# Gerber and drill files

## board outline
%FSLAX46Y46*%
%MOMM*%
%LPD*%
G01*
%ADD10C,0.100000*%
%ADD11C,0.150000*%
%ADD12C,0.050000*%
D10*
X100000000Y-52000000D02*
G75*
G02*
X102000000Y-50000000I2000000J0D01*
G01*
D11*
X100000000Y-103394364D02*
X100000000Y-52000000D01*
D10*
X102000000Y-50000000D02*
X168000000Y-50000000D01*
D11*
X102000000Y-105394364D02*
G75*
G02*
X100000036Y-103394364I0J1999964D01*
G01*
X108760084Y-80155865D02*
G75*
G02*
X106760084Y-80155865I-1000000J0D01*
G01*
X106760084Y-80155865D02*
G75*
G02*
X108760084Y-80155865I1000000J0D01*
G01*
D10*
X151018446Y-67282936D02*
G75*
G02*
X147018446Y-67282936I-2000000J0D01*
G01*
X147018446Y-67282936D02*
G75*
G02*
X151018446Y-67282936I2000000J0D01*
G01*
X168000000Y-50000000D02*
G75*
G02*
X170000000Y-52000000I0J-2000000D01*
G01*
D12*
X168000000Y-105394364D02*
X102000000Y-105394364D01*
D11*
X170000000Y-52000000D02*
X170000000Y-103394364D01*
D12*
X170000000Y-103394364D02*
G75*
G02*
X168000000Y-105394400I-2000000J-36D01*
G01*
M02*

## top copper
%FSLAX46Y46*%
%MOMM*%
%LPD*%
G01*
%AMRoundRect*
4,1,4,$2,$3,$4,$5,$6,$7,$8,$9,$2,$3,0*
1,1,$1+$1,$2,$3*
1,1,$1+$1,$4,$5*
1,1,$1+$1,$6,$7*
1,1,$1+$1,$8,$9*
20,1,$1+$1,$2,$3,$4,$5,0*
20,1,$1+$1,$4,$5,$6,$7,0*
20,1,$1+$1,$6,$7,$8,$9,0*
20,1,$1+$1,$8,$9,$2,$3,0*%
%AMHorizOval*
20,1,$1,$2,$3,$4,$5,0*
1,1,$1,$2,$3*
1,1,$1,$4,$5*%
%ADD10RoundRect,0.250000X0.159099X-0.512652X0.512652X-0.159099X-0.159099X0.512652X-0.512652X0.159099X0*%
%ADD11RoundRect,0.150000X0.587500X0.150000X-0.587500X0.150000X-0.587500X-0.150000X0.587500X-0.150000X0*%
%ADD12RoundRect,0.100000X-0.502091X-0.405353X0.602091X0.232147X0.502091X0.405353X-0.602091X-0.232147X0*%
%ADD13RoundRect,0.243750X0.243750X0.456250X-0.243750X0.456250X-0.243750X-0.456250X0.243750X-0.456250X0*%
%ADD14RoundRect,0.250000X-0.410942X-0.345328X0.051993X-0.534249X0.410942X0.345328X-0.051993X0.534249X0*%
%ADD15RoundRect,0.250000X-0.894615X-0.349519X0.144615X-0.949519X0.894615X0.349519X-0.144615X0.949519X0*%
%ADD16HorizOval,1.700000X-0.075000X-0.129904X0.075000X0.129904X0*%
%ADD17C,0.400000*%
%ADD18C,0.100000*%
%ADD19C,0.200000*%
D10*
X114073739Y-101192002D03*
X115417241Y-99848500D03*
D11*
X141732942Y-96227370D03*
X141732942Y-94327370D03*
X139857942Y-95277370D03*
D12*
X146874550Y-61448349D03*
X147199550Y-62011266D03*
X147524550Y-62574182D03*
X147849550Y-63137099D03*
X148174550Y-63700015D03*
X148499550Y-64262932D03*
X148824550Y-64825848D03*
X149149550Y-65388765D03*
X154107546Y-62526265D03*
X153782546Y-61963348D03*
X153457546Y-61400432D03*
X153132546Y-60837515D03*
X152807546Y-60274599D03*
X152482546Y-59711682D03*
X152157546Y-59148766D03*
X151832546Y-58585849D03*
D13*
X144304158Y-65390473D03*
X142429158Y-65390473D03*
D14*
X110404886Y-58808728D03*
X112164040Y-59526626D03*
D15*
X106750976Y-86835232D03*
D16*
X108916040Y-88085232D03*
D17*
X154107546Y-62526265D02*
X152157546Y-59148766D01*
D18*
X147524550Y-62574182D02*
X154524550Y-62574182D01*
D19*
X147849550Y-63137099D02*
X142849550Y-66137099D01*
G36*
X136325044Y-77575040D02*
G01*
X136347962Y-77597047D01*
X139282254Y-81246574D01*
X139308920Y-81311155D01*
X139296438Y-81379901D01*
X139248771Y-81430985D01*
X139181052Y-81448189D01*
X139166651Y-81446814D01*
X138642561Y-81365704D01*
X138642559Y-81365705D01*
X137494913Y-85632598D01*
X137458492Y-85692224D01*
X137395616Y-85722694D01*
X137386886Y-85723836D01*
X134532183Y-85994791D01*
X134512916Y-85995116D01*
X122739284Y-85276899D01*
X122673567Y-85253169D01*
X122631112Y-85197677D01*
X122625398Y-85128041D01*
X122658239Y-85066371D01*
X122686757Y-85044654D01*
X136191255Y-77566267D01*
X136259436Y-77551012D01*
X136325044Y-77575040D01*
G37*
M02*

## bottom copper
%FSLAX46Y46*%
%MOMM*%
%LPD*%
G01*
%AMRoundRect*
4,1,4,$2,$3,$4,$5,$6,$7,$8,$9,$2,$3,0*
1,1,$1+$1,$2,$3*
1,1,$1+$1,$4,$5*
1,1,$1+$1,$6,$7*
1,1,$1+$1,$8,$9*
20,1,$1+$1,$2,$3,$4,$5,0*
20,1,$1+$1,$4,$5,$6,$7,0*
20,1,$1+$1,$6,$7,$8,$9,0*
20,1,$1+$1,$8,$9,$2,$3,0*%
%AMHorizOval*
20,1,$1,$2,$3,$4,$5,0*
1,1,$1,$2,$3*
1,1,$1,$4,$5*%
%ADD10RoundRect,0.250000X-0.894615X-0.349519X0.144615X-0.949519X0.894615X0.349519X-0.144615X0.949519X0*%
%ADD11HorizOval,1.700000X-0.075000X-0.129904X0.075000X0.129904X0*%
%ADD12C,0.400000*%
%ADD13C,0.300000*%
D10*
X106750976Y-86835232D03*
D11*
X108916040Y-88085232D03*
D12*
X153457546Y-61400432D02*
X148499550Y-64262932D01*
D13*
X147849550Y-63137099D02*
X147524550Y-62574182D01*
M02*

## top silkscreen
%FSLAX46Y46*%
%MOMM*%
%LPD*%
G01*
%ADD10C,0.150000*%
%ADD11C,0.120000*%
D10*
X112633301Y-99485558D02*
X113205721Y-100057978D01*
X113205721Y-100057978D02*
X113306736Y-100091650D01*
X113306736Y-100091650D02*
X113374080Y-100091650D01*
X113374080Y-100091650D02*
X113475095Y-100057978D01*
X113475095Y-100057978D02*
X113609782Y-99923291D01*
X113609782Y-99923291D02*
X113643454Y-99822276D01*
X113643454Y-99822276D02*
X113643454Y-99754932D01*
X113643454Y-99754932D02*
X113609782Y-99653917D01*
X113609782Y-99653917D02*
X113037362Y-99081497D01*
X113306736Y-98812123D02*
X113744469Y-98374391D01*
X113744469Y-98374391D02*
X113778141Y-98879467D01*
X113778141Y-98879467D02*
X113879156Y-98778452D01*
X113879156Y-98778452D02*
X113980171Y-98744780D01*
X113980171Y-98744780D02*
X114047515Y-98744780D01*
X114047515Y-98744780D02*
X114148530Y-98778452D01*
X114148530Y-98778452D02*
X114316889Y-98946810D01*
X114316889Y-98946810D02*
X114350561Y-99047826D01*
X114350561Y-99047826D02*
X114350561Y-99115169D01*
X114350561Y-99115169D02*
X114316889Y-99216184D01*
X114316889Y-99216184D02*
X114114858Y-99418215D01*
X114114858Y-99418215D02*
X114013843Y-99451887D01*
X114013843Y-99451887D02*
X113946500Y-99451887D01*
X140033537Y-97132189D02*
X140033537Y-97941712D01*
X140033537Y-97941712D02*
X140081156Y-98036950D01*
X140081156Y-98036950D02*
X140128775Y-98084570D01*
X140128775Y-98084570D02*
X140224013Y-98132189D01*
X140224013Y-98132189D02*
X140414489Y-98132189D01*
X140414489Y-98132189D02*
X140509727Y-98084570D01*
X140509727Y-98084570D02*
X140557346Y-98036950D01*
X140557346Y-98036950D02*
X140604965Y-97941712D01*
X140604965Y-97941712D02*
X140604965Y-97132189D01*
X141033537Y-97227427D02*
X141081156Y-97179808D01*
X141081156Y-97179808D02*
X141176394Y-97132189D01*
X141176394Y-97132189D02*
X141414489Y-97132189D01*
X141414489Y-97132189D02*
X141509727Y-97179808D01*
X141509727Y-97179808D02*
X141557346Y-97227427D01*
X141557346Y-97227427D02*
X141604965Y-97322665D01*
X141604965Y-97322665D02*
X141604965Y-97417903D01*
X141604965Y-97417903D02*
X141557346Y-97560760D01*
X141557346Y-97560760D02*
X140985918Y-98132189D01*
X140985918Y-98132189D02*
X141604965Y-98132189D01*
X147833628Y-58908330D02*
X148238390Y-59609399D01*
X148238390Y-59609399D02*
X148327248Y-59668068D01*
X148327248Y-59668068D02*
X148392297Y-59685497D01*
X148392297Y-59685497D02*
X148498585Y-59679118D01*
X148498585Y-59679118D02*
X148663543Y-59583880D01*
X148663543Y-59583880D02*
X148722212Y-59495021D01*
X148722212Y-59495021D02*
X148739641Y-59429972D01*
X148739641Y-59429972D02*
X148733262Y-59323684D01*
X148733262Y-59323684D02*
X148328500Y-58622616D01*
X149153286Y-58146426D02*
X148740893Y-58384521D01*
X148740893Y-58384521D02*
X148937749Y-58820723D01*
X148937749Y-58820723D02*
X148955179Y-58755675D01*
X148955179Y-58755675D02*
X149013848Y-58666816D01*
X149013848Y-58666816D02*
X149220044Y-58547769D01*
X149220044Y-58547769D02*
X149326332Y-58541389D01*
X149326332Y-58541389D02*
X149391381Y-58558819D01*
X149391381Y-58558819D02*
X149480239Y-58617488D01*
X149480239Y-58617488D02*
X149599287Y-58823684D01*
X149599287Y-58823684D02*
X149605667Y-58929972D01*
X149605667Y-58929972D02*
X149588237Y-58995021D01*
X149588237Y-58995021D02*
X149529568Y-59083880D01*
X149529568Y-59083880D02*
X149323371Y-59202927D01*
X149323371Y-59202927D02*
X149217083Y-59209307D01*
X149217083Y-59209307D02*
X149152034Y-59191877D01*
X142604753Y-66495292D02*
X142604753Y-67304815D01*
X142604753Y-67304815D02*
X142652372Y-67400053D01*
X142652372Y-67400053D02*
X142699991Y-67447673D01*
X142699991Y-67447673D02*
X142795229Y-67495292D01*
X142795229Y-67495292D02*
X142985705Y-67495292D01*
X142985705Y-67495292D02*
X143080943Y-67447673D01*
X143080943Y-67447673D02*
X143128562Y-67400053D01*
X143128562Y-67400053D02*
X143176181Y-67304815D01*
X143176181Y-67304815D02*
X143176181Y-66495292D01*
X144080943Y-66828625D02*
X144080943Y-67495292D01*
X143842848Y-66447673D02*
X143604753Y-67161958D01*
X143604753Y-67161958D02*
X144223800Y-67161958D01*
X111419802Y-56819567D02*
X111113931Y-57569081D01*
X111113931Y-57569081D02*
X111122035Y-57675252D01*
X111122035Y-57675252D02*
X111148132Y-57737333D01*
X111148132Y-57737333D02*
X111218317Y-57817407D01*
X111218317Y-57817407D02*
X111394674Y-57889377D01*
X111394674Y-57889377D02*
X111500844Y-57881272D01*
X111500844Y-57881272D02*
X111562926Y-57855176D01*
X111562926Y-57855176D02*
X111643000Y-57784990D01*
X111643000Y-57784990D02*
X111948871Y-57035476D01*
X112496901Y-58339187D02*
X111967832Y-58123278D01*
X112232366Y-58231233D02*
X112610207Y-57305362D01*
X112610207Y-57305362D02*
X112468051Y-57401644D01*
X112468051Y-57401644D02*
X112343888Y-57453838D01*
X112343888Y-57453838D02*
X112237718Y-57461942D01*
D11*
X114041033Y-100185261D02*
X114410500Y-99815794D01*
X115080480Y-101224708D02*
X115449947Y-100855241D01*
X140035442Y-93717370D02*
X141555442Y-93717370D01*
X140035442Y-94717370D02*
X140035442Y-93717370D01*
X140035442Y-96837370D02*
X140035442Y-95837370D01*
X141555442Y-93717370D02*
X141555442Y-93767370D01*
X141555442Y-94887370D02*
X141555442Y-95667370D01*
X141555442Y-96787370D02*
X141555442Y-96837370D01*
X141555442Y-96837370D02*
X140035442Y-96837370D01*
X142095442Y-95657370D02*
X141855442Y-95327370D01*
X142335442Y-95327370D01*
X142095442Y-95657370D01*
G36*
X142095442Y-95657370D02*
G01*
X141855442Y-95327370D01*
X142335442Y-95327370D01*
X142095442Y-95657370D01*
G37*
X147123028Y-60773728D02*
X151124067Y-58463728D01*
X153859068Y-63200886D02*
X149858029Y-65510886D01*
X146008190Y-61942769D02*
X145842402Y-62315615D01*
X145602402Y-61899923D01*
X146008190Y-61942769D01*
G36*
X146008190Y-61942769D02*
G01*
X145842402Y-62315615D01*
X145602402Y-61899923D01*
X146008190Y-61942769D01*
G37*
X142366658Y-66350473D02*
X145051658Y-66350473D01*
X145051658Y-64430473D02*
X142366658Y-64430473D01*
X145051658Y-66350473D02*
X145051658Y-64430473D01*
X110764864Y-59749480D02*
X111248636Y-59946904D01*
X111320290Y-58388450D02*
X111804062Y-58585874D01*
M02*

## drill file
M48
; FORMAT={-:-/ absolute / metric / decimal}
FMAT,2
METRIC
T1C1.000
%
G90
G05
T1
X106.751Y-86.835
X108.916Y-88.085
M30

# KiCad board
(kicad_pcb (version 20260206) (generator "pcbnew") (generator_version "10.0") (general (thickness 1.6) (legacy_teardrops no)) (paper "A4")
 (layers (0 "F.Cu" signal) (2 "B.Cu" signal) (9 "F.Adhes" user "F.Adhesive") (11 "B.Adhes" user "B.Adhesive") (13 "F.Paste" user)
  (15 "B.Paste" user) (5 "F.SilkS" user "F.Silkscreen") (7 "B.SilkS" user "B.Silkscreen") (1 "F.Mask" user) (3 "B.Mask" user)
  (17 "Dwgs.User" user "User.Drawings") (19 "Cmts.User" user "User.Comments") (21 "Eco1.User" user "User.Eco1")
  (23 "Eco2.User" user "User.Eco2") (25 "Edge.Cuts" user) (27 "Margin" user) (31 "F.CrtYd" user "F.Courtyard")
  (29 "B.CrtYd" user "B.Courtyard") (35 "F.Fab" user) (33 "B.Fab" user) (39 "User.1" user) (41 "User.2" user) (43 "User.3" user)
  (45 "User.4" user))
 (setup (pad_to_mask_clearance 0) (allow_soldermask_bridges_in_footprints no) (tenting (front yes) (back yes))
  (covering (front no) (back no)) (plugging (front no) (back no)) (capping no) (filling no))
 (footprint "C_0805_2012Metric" (layer "F.Cu") (at 114.74549 100.520251 45)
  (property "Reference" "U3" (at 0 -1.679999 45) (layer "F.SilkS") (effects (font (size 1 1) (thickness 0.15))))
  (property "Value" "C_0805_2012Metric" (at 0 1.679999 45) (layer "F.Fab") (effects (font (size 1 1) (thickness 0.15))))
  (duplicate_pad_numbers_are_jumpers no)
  (fp_line (start -0.261253 -0.735) (end 0.261253 -0.735) (stroke (width 0.12) (type solid)) (layer "F.SilkS"))
  (fp_line (start -0.261253 0.735) (end 0.261253 0.735) (stroke (width 0.12) (type solid)) (layer "F.SilkS"))
  (pad "1" smd roundrect (at -0.949999 0 45) (size 1 1.45) (layers "F.Cu" "F.Mask" "F.Paste") (roundrect_rratio 0.25) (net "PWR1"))
  (pad "2" smd roundrect (at 0.949999 0 45) (size 1 1.45) (layers "F.Cu" "F.Mask" "F.Paste") (roundrect_rratio 0.25) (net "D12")))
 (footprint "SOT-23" (layer "F.Cu") (at 140.795442 95.27737 180)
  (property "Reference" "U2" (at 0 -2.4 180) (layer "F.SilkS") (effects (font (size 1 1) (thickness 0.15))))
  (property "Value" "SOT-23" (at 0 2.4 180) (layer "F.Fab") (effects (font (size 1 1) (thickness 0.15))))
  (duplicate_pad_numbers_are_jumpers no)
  (fp_line (start 0.76 1.56) (end -0.76 1.56) (stroke (width 0.12) (type solid)) (layer "F.SilkS"))
  (fp_line (start 0.76 0.56) (end 0.76 1.56) (stroke (width 0.12) (type solid)) (layer "F.SilkS"))
  (fp_line (start 0.76 -1.56) (end 0.76 -0.56) (stroke (width 0.12) (type solid)) (layer "F.SilkS"))
  (fp_line (start -0.76 1.56) (end -0.76 1.51) (stroke (width 0.12) (type solid)) (layer "F.SilkS"))
  (fp_line (start -0.76 0.39) (end -0.76 -0.39) (stroke (width 0.12) (type solid)) (layer "F.SilkS"))
  (fp_line (start -0.76 -1.51) (end -0.76 -1.56) (stroke (width 0.12) (type solid)) (layer "F.SilkS"))
  (fp_line (start -0.76 -1.56) (end 0.76 -1.56) (stroke (width 0.12) (type solid)) (layer "F.SilkS"))
  (fp_poly (pts (xy -1.3 -0.38) (xy -1.06 -0.05) (xy -1.54 -0.05)) (stroke (width 0.12) (type solid)) (fill yes) (layer "F.SilkS"))
  (pad "1" smd roundrect (at -0.9375 -0.95 180) (size 1.475 0.6) (layers "F.Cu" "F.Mask" "F.Paste") (roundrect_rratio 0.25) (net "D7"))
  (pad "2" smd roundrect (at -0.9375 0.95 180) (size 1.475 0.6) (layers "F.Cu" "F.Mask" "F.Paste") (roundrect_rratio 0.25) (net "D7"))
  (pad "3" smd roundrect (at 0.9375 0 180) (size 1.475 0.6) (layers "F.Cu" "F.Mask" "F.Paste") (roundrect_rratio 0.25) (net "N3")))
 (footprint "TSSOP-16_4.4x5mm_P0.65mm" (layer "F.Cu") (at 150.491048 61.987307 30)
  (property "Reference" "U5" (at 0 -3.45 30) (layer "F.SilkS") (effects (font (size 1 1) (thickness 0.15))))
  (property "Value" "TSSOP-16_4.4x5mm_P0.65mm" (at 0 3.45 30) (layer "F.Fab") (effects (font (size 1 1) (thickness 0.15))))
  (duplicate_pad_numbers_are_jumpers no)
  (fp_line (start -2.310001 -2.735) (end 2.31 -2.734999) (stroke (width 0.12) (type solid)) (layer "F.SilkS"))
  (fp_line (start 2.310001 2.735) (end -2.31 2.734999) (stroke (width 0.12) (type solid)) (layer "F.SilkS"))
  (fp_poly (pts (xy -3.86 -2.28) (xy -4.19 -2.04) (xy -4.19 -2.52)) (stroke (width 0.12) (type solid)) (fill yes) (layer "F.SilkS"))
  (pad "1" smd roundrect (at -2.8625 -2.275 30) (size 1.475 0.4) (layers "F.Cu" "F.Mask" "F.Paste") (roundrect_rratio 0.25) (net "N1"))
  (pad "2" smd roundrect (at -2.8625 -1.625 30) (size 1.475 0.4) (layers "F.Cu" "F.Mask" "F.Paste") (roundrect_rratio 0.25) (clearance 0.1))
  (pad "3" smd roundrect (at -2.8625 -0.975 30) (size 1.475 0.4) (layers "F.Cu" "F.Mask" "F.Paste") (roundrect_rratio 0.25))
  (pad "4" smd roundrect (at -2.8625 -0.325 30) (size 1.475 0.4) (layers "F.Cu" "F.Mask" "F.Paste") (roundrect_rratio 0.25) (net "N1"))
  (pad "5" smd roundrect (at -2.8625 0.325 30) (size 1.475 0.4) (layers "F.Cu" "F.Mask" "F.Paste") (roundrect_rratio 0.25) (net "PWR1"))
  (pad "6" smd roundrect (at -2.8625 0.975 30) (size 1.475 0.4) (layers "F.Cu" "F.Mask" "F.Paste") (roundrect_rratio 0.25) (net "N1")
   (clearance 0.1))
  (pad "7" smd roundrect (at -2.8625 1.625 30) (size 1.475 0.4) (layers "F.Cu" "F.Mask" "F.Paste") (roundrect_rratio 0.25) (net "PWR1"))
  (pad "8" smd roundrect (at -2.8625 2.275 30) (size 1.475 0.4) (layers "F.Cu" "F.Mask" "F.Paste") (roundrect_rratio 0.25) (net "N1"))
  (pad "9" smd roundrect (at 2.8625 2.275 30) (size 1.475 0.4) (layers "F.Cu" "F.Mask" "F.Paste") (roundrect_rratio 0.25))
  (pad "10" smd roundrect (at 2.8625 1.625 30) (size 1.475 0.4) (layers "F.Cu" "F.Mask" "F.Paste") (roundrect_rratio 0.25))
  (pad "11" smd roundrect (at 2.8625 0.975 30) (size 1.475 0.4) (layers "F.Cu" "F.Mask" "F.Paste") (roundrect_rratio 0.25))
  (pad "12" smd roundrect (at 2.8625 0.325 30) (size 1.475 0.4) (layers "F.Cu" "F.Mask" "F.Paste") (roundrect_rratio 0.25) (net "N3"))
  (pad "13" smd roundrect (at 2.8625 -0.325 30) (size 1.475 0.4) (layers "F.Cu" "F.Mask" "F.Paste") (roundrect_rratio 0.25) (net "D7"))
  (pad "14" smd roundrect (at 2.8625 -0.975 30) (size 1.475 0.4) (layers "F.Cu" "F.Mask" "F.Paste") (roundrect_rratio 0.25) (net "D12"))
  (pad "15" smd roundrect (at 2.8625 -1.625 30) (size 1.475 0.4) (layers "F.Cu" "F.Mask" "F.Paste") (roundrect_rratio 0.25))
  (pad "16" smd roundrect (at 2.8625 -2.275 30) (size 1.475 0.4) (layers "F.Cu" "F.Mask" "F.Paste") (roundrect_rratio 0.25) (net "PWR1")))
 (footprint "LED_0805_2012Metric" (layer "F.Cu") (at 143.366658 65.390473 180)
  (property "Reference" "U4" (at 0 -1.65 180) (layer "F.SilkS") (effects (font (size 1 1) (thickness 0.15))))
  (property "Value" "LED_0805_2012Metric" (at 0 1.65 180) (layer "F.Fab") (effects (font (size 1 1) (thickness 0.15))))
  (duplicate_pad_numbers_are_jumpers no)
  (fp_line (start 1 -0.96) (end -1.685 -0.96) (stroke (width 0.12) (type solid)) (layer "F.SilkS"))
  (fp_line (start -1.685 0.96) (end 1 0.96) (stroke (width 0.12) (type solid)) (layer "F.SilkS"))
  (fp_line (start -1.685 -0.96) (end -1.685 0.96) (stroke (width 0.12) (type solid)) (layer "F.SilkS"))
  (pad "1" smd roundrect (at -0.9375 0 180) (size 0.975 1.4) (layers "F.Cu" "F.Mask" "F.Paste") (roundrect_rratio 0.25) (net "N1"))
  (pad "2" smd roundrect (at 0.9375 0 180) (size 0.975 1.4) (layers "F.Cu" "F.Mask" "F.Paste") (roundrect_rratio 0.25) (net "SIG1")))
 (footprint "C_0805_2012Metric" (layer "F.Cu") (at 111.284463 59.167677 -22.2)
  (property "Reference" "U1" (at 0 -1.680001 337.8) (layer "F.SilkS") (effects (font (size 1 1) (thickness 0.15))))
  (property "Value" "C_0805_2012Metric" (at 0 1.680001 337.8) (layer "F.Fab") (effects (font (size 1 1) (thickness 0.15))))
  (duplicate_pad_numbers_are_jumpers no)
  (fp_line (start -0.261253 0.735) (end 0.261253 0.735) (stroke (width 0.12) (type solid)) (layer "F.SilkS"))
  (fp_line (start -0.261253 -0.735) (end 0.261253 -0.735) (stroke (width 0.12) (type solid)) (layer "F.SilkS"))
  (pad "1" smd roundrect (at -0.95 0 337.8) (size 1 1.45) (layers "F.Cu" "F.Mask" "F.Paste") (roundrect_rratio 0.25) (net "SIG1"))
  (pad "2" smd roundrect (at 0.95 0 337.8) (size 1 1.45) (layers "F.Cu" "F.Mask" "F.Paste") (roundrect_rratio 0.25)))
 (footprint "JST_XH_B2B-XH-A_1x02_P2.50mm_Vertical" (layer "B.Cu") (at 106.750976 86.835232 -30)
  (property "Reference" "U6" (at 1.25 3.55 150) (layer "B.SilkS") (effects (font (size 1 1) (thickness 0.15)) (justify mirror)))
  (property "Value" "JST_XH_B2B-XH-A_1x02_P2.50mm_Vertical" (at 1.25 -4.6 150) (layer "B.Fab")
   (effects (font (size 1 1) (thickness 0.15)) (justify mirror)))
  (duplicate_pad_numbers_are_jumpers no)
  (pad "1" thru_hole roundrect (at 0 0 330) (size 1.7 2) (drill 1) (layers "*.Cu" "*.Mask") (remove_unused_layers no)
   (roundrect_rratio 0.147059) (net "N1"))
  (pad "2" thru_hole oval (at 2.5 0 330) (size 1.7 2) (drill 1) (layers "*.Cu" "*.Mask") (remove_unused_layers no) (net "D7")
   (clearance 0.1)))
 (gr_arc (start 100 52) (mid 100.585786 50.585786) (end 102 50) (stroke (width 0.1) (type default)) (layer "Edge.Cuts"))
 (gr_line (start 100 103.394364) (end 100 52) (stroke (width 0.15) (type default)) (layer "Edge.Cuts"))
 (gr_line (start 102 50) (end 168 50) (stroke (width 0.1) (type default)) (layer "Edge.Cuts"))
 (gr_arc (start 102 105.394364) (mid 100.585786 104.808577) (end 100 103.394364) (stroke (width 0.15) (type default)) (layer "Edge.Cuts"))
 (gr_circle (center 107.760084 80.155865) (end 108.760084 80.155865) (stroke (width 0.15) (type default)) (fill no) (layer "Edge.Cuts"))
 (gr_circle (center 149.018446 67.282936) (end 151.018446 67.282936) (stroke (width 0.1) (type default)) (fill no) (layer "Edge.Cuts"))
 (gr_arc (start 168 50) (mid 169.414213 50.585786) (end 170 52) (stroke (width 0.1) (type default)) (layer "Edge.Cuts"))
 (gr_line (start 168 105.394364) (end 102 105.394364) (stroke (width 0.05) (type default)) (layer "Edge.Cuts"))
 (gr_line (start 170 52) (end 170 103.394364) (stroke (width 0.15) (type default)) (layer "Edge.Cuts"))
 (gr_arc (start 170 103.394364) (mid 169.414213 104.808577) (end 168 105.394364) (stroke (width 0.05) (type default)) (layer "Edge.Cuts"))
 (segment (start 154.107546 62.526265) (end 152.157546 59.148766) (width 0.4) (layer "F.Cu") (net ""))
 (segment (start 147.52455 62.574182) (end 154.52455 62.574182) (width 0.1) (layer "F.Cu") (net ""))
 (segment (start 153.457546 61.400432) (end 148.49955 64.262932) (width 0.4) (layer "B.Cu") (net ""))
 (segment (start 147.84955 63.137099) (end 142.84955 66.137099) (width 0.2) (layer "F.Cu") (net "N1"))
 (segment (start 147.84955 63.137099) (end 147.52455 62.574182) (width 0.3) (layer "B.Cu") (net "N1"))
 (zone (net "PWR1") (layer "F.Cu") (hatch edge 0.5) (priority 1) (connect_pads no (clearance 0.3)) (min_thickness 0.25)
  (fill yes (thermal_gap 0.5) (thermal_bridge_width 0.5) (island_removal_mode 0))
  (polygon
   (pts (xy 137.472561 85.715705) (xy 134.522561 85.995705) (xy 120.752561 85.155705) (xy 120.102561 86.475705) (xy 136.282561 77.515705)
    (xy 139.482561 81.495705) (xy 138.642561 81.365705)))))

